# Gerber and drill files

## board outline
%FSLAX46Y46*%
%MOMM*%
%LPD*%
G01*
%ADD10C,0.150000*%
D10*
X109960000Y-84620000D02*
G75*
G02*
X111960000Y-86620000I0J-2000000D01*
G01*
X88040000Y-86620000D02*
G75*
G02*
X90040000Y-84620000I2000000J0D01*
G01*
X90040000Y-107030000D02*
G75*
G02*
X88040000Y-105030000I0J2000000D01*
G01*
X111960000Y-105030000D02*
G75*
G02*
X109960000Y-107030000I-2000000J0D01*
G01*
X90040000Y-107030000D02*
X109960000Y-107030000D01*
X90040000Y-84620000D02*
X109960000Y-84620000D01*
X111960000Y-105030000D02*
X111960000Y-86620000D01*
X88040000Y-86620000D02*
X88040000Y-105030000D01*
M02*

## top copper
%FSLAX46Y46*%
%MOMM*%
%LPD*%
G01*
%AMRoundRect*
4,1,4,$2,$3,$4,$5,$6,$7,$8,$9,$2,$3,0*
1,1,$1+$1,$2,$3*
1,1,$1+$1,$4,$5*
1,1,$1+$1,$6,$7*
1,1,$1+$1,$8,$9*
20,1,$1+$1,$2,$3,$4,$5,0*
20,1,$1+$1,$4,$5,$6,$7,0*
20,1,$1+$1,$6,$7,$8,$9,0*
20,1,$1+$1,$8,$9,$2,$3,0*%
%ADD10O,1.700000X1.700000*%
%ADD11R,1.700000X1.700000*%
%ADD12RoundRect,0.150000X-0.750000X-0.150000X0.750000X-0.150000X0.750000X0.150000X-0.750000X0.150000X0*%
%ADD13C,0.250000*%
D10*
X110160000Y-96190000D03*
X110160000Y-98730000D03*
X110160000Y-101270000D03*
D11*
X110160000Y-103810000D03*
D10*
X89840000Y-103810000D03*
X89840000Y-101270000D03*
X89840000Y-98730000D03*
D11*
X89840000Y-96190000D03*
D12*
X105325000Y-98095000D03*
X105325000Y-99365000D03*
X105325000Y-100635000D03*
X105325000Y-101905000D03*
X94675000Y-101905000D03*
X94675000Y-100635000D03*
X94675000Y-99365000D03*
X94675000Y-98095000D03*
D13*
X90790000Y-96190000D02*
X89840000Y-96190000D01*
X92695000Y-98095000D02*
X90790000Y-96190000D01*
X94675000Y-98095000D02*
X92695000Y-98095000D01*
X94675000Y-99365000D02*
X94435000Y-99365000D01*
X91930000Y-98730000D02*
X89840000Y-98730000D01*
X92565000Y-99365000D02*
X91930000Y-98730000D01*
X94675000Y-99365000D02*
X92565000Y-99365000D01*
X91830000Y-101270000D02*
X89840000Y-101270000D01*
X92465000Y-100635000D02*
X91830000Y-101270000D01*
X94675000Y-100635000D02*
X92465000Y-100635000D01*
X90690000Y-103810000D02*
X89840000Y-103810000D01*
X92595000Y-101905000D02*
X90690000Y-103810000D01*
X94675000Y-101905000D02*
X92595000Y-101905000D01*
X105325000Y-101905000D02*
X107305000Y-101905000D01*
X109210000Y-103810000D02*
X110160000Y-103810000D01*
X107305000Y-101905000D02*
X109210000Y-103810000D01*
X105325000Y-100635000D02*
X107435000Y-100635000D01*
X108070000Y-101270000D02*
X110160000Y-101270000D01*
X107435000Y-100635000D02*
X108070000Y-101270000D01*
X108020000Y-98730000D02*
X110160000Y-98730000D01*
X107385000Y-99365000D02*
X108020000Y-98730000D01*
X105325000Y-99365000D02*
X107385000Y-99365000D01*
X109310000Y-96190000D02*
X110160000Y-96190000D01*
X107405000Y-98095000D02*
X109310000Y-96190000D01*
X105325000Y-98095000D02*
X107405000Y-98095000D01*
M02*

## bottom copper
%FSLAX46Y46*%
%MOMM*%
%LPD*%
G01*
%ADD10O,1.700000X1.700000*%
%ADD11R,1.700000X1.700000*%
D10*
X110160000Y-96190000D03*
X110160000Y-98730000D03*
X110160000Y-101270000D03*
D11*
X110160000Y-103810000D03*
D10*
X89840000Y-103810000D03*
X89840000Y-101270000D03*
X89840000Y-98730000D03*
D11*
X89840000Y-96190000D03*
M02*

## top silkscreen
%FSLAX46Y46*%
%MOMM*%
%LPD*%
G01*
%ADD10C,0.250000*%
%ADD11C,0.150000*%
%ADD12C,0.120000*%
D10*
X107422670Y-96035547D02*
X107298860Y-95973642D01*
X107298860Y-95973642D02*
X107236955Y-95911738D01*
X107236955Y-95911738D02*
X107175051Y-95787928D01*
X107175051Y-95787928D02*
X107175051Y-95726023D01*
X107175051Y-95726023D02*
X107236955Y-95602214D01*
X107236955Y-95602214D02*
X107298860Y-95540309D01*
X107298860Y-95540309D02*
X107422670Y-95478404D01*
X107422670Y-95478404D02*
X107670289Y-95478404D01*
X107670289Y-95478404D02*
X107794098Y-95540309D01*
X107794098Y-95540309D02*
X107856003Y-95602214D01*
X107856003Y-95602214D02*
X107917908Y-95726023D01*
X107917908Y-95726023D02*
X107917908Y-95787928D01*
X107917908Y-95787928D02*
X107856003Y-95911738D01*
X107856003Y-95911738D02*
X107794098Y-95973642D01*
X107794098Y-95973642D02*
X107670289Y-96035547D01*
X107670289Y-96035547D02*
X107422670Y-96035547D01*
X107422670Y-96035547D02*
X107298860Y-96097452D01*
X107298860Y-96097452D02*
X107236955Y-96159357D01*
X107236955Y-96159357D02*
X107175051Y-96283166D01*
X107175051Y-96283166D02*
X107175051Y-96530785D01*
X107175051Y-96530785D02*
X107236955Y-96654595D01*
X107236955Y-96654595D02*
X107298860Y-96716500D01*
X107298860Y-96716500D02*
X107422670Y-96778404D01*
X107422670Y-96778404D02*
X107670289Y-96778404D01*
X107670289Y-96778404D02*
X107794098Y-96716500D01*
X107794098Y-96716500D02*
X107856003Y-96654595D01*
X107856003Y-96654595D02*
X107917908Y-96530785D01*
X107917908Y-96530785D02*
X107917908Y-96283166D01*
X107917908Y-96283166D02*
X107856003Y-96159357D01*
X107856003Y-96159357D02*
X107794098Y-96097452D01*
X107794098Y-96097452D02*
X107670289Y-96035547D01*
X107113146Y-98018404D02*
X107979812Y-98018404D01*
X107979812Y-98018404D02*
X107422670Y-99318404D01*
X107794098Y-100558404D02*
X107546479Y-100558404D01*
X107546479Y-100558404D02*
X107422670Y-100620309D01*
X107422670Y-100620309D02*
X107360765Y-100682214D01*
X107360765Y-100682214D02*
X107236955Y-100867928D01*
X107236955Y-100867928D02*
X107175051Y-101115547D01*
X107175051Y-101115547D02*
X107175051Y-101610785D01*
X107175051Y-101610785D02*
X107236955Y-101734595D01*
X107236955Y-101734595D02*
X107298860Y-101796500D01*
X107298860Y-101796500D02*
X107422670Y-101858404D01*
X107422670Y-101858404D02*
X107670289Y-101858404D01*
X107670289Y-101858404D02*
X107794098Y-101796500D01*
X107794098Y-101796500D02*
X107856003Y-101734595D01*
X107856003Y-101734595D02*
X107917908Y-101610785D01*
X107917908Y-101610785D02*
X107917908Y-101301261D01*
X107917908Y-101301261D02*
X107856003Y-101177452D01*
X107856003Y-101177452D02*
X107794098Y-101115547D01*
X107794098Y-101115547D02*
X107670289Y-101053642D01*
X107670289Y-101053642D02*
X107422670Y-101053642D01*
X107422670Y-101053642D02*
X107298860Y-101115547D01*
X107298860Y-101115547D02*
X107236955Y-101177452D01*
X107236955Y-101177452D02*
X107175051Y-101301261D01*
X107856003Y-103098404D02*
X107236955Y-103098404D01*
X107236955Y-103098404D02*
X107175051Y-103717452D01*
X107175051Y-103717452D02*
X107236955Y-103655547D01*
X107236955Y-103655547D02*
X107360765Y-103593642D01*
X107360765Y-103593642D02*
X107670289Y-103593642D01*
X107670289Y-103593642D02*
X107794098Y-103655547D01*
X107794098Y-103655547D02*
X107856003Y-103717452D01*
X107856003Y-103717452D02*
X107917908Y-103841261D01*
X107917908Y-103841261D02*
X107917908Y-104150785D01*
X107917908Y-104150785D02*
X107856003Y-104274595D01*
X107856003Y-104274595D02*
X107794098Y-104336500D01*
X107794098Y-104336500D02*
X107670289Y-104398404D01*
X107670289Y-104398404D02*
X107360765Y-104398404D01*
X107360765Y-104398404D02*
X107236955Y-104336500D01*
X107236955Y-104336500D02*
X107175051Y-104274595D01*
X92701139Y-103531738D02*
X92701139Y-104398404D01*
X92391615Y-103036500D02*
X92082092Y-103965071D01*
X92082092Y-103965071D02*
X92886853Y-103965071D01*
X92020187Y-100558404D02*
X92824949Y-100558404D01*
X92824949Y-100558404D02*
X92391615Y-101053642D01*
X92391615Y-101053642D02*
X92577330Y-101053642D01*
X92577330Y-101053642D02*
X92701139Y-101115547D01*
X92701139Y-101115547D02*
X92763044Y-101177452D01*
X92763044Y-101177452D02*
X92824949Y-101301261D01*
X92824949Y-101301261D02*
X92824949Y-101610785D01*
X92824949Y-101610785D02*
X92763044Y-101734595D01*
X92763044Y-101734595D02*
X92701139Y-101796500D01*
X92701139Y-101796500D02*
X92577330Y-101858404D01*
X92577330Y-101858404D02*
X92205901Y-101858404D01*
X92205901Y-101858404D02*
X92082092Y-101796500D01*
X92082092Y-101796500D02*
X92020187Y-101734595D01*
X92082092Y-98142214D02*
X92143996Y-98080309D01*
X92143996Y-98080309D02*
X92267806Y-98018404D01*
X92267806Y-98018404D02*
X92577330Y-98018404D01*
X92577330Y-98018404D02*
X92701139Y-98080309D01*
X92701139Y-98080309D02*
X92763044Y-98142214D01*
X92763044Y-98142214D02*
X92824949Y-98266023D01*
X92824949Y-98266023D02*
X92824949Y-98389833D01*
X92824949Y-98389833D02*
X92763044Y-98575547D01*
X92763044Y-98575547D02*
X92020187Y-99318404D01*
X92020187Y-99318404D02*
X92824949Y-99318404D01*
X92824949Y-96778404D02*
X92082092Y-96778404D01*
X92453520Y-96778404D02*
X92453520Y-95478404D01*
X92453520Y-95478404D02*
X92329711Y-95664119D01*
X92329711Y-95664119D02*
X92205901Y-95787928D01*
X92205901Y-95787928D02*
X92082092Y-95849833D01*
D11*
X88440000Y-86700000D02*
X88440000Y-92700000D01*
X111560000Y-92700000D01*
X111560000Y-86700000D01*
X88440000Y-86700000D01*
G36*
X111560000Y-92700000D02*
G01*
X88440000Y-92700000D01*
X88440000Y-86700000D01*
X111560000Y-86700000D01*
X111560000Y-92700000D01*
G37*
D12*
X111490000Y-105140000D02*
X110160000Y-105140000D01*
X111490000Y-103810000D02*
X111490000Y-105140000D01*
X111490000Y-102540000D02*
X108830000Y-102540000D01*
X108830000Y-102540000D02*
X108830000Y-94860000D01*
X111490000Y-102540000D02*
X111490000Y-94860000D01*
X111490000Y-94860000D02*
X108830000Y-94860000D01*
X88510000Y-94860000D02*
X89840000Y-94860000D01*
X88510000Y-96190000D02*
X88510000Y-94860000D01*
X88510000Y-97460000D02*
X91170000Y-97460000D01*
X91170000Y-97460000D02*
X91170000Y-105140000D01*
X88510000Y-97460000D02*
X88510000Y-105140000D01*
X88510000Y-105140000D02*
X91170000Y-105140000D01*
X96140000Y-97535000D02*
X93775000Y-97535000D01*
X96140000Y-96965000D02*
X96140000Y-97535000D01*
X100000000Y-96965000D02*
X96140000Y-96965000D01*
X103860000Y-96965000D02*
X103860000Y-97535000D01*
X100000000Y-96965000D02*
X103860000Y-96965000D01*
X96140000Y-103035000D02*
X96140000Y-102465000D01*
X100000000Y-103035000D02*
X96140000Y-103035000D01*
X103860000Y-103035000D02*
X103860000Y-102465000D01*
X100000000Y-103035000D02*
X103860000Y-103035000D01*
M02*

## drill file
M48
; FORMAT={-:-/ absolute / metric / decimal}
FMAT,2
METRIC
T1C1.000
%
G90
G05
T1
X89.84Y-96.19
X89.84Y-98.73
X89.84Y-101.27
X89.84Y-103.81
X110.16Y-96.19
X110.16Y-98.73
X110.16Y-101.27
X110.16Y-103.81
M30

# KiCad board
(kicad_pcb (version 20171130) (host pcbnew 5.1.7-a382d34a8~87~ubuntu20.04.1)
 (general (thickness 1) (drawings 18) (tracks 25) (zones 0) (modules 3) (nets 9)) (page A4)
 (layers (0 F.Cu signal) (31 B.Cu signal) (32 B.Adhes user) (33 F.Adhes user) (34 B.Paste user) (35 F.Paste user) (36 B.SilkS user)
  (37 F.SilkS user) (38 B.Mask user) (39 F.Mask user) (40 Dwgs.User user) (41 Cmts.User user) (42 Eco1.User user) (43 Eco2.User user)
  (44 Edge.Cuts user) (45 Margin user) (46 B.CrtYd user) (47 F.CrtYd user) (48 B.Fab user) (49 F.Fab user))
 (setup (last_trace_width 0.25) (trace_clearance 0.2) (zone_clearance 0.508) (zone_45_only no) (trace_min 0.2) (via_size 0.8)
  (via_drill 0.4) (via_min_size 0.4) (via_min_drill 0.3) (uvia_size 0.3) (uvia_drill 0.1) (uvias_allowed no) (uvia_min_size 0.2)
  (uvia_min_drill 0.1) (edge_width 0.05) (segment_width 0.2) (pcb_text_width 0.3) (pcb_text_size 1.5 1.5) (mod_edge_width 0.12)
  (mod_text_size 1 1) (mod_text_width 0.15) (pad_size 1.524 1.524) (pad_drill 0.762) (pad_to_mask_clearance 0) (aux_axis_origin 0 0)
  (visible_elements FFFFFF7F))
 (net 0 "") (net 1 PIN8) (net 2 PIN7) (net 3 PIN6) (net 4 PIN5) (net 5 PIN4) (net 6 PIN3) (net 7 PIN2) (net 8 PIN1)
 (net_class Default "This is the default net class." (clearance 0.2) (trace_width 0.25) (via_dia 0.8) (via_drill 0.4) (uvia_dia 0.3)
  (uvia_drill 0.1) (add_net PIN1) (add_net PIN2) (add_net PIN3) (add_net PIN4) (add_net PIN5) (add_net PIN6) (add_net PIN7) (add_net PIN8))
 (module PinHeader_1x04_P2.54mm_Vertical (layer F.Cu) (at 110.16 103.81 180)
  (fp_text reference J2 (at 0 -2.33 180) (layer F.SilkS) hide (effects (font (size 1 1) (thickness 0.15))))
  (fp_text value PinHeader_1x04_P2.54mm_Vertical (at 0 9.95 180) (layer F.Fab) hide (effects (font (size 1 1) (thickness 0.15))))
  (fp_line (start -1.33 -1.33) (end 0 -1.33) (layer F.SilkS) (width 0.12))
  (fp_line (start -1.33 0) (end -1.33 -1.33) (layer F.SilkS) (width 0.12))
  (fp_line (start -1.33 1.27) (end 1.33 1.27) (layer F.SilkS) (width 0.12))
  (fp_line (start 1.33 1.27) (end 1.33 8.95) (layer F.SilkS) (width 0.12))
  (fp_line (start -1.33 1.27) (end -1.33 8.95) (layer F.SilkS) (width 0.12))
  (fp_line (start -1.33 8.95) (end 1.33 8.95) (layer F.SilkS) (width 0.12))
  (pad 4 thru_hole oval (at 0 7.62 180) (size 1.7 1.7) (drill 1) (layers *.Cu *.Mask) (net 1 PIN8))
  (pad 3 thru_hole oval (at 0 5.08 180) (size 1.7 1.7) (drill 1) (layers *.Cu *.Mask) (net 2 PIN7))
  (pad 2 thru_hole oval (at 0 2.54 180) (size 1.7 1.7) (drill 1) (layers *.Cu *.Mask) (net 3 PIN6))
  (pad 1 thru_hole rect (at 0 0 180) (size 1.7 1.7) (drill 1) (layers *.Cu *.Mask) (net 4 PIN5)))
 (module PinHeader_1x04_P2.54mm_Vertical (layer F.Cu) (at 89.84 96.19)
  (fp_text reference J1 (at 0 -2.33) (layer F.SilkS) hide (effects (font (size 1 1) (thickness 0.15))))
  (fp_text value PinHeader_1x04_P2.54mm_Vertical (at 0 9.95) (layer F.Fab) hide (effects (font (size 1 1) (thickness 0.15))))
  (fp_line (start -1.33 -1.33) (end 0 -1.33) (layer F.SilkS) (width 0.12))
  (fp_line (start -1.33 0) (end -1.33 -1.33) (layer F.SilkS) (width 0.12))
  (fp_line (start -1.33 1.27) (end 1.33 1.27) (layer F.SilkS) (width 0.12))
  (fp_line (start 1.33 1.27) (end 1.33 8.95) (layer F.SilkS) (width 0.12))
  (fp_line (start -1.33 1.27) (end -1.33 8.95) (layer F.SilkS) (width 0.12))
  (fp_line (start -1.33 8.95) (end 1.33 8.95) (layer F.SilkS) (width 0.12))
  (pad 4 thru_hole oval (at 0 7.62) (size 1.7 1.7) (drill 1) (layers *.Cu *.Mask) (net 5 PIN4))
  (pad 3 thru_hole oval (at 0 5.08) (size 1.7 1.7) (drill 1) (layers *.Cu *.Mask) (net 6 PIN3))
  (pad 2 thru_hole oval (at 0 2.54) (size 1.7 1.7) (drill 1) (layers *.Cu *.Mask) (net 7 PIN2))
  (pad 1 thru_hole rect (at 0 0) (size 1.7 1.7) (drill 1) (layers *.Cu *.Mask) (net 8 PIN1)))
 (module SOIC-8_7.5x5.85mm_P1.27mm (layer F.Cu) (at 100 100)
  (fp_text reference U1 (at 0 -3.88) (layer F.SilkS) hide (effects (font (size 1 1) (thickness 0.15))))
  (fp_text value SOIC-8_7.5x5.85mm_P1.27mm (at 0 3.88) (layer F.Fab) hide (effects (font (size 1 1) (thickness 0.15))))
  (fp_line (start -3.86 -2.465) (end -6.225 -2.465) (layer F.SilkS) (width 0.12))
  (fp_line (start -3.86 -3.035) (end -3.86 -2.465) (layer F.SilkS) (width 0.12))
  (fp_line (start 0 -3.035) (end -3.86 -3.035) (layer F.SilkS) (width 0.12))
  (fp_line (start 3.86 -3.035) (end 3.86 -2.465) (layer F.SilkS) (width 0.12))
  (fp_line (start 0 -3.035) (end 3.86 -3.035) (layer F.SilkS) (width 0.12))
  (fp_line (start -3.86 3.035) (end -3.86 2.465) (layer F.SilkS) (width 0.12))
  (fp_line (start 0 3.035) (end -3.86 3.035) (layer F.SilkS) (width 0.12))
  (fp_line (start 3.86 3.035) (end 3.86 2.465) (layer F.SilkS) (width 0.12))
  (fp_line (start 0 3.035) (end 3.86 3.035) (layer F.SilkS) (width 0.12))
  (pad 8 smd roundrect (at 5.325 -1.905) (size 1.8 0.6) (layers F.Cu F.Paste F.Mask) (roundrect_rratio 0.25) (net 1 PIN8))
  (pad 7 smd roundrect (at 5.325 -0.635) (size 1.8 0.6) (layers F.Cu F.Paste F.Mask) (roundrect_rratio 0.25) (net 2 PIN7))
  (pad 6 smd roundrect (at 5.325 0.635) (size 1.8 0.6) (layers F.Cu F.Paste F.Mask) (roundrect_rratio 0.25) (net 3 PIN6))
  (pad 5 smd roundrect (at 5.325 1.905) (size 1.8 0.6) (layers F.Cu F.Paste F.Mask) (roundrect_rratio 0.25) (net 4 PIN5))
  (pad 4 smd roundrect (at -5.325 1.905) (size 1.8 0.6) (layers F.Cu F.Paste F.Mask) (roundrect_rratio 0.25) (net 5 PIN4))
  (pad 3 smd roundrect (at -5.325 0.635) (size 1.8 0.6) (layers F.Cu F.Paste F.Mask) (roundrect_rratio 0.25) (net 6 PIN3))
  (pad 2 smd roundrect (at -5.325 -0.635) (size 1.8 0.6) (layers F.Cu F.Paste F.Mask) (roundrect_rratio 0.25) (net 7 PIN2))
  (pad 1 smd roundrect (at -5.325 -1.905) (size 1.8 0.6) (layers F.Cu F.Paste F.Mask) (roundrect_rratio 0.25) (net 8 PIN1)))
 (gr_arc (start 109.96 86.62) (end 109.96 84.62) (angle 90) (layer Edge.Cuts) (width 0.15))
 (gr_arc (start 90.04 86.62) (end 88.04 86.62) (angle 90) (layer Edge.Cuts) (width 0.15))
 (gr_arc (start 90.04 105.03) (end 90.04 107.03) (angle 90) (layer Edge.Cuts) (width 0.15))
 (gr_arc (start 109.96 105.03) (end 111.96 105.03) (angle 90) (layer Edge.Cuts) (width 0.15))
 (gr_line (start 90.04 107.03) (end 109.96 107.03) (layer Edge.Cuts) (width 0.15))
 (gr_line (start 90.04 84.62) (end 109.96 84.62) (layer Edge.Cuts) (width 0.15))
 (gr_line (start 111.96 105.03) (end 111.96 86.62) (layer Edge.Cuts) (width 0.15))
 (gr_line (start 88.04 86.62) (end 88.04 105.03) (layer Edge.Cuts) (width 0.15))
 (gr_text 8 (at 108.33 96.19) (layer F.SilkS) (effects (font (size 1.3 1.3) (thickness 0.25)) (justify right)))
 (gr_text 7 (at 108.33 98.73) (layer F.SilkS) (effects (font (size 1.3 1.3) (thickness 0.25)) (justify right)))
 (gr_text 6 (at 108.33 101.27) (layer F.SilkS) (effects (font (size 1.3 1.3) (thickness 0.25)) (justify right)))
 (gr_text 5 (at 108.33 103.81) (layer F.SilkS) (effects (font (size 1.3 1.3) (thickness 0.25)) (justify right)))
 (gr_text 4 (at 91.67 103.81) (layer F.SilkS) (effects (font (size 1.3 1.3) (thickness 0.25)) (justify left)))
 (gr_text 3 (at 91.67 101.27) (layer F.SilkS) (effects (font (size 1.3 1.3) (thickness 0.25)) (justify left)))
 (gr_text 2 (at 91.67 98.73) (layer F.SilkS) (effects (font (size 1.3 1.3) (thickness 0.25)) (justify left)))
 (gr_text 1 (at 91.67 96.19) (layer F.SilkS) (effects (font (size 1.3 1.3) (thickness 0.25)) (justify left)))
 (gr_poly (pts (xy 88.44 86.7) (xy 88.44 92.7) (xy 111.56 92.7) (xy 111.56 86.7)) (layer F.SilkS) (width 0.15))
 (segment (start 90.79 96.19) (end 89.84 96.19) (width 0.25) (layer F.Cu) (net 8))
 (segment (start 92.695 98.095) (end 90.79 96.19) (width 0.25) (layer F.Cu) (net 8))
 (segment (start 94.675 98.095) (end 92.695 98.095) (width 0.25) (layer F.Cu) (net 8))
 (segment (start 94.675 99.365) (end 94.435 99.365) (width 0.25) (layer F.Cu) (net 7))
 (segment (start 91.93 98.73) (end 89.84 98.73) (width 0.25) (layer F.Cu) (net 7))
 (segment (start 92.565 99.365) (end 91.93 98.73) (width 0.25) (layer F.Cu) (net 7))
 (segment (start 94.675 99.365) (end 92.565 99.365) (width 0.25) (layer F.Cu) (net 7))
 (segment (start 91.83 101.27) (end 89.84 101.27) (width 0.25) (layer F.Cu) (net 6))
 (segment (start 92.465 100.635) (end 91.83 101.27) (width 0.25) (layer F.Cu) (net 6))
 (segment (start 94.675 100.635) (end 92.465 100.635) (width 0.25) (layer F.Cu) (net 6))
 (segment (start 90.69 103.81) (end 89.84 103.81) (width 0.25) (layer F.Cu) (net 5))
 (segment (start 92.595 101.905) (end 90.69 103.81) (width 0.25) (layer F.Cu) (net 5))
 (segment (start 94.675 101.905) (end 92.595 101.905) (width 0.25) (layer F.Cu) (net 5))
 (segment (start 105.325 101.905) (end 107.305 101.905) (width 0.25) (layer F.Cu) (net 4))
 (segment (start 109.21 103.81) (end 110.16 103.81) (width 0.25) (layer F.Cu) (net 4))
 (segment (start 107.305 101.905) (end 109.21 103.81) (width 0.25) (layer F.Cu) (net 4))
 (segment (start 105.325 100.635) (end 107.435 100.635) (width 0.25) (layer F.Cu) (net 3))
 (segment (start 108.07 101.27) (end 110.16 101.27) (width 0.25) (layer F.Cu) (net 3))
 (segment (start 107.435 100.635) (end 108.07 101.27) (width 0.25) (layer F.Cu) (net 3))
 (segment (start 108.02 98.73) (end 110.16 98.73) (width 0.25) (layer F.Cu) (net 2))
 (segment (start 107.385 99.365) (end 108.02 98.73) (width 0.25) (layer F.Cu) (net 2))
 (segment (start 105.325 99.365) (end 107.385 99.365) (width 0.25) (layer F.Cu) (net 2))
 (segment (start 109.31 96.19) (end 110.16 96.19) (width 0.25) (layer F.Cu) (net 1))
 (segment (start 107.405 98.095) (end 109.31 96.19) (width 0.25) (layer F.Cu) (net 1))
 (segment (start 105.325 98.095) (end 107.405 98.095) (width 0.25) (layer F.Cu) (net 1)))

